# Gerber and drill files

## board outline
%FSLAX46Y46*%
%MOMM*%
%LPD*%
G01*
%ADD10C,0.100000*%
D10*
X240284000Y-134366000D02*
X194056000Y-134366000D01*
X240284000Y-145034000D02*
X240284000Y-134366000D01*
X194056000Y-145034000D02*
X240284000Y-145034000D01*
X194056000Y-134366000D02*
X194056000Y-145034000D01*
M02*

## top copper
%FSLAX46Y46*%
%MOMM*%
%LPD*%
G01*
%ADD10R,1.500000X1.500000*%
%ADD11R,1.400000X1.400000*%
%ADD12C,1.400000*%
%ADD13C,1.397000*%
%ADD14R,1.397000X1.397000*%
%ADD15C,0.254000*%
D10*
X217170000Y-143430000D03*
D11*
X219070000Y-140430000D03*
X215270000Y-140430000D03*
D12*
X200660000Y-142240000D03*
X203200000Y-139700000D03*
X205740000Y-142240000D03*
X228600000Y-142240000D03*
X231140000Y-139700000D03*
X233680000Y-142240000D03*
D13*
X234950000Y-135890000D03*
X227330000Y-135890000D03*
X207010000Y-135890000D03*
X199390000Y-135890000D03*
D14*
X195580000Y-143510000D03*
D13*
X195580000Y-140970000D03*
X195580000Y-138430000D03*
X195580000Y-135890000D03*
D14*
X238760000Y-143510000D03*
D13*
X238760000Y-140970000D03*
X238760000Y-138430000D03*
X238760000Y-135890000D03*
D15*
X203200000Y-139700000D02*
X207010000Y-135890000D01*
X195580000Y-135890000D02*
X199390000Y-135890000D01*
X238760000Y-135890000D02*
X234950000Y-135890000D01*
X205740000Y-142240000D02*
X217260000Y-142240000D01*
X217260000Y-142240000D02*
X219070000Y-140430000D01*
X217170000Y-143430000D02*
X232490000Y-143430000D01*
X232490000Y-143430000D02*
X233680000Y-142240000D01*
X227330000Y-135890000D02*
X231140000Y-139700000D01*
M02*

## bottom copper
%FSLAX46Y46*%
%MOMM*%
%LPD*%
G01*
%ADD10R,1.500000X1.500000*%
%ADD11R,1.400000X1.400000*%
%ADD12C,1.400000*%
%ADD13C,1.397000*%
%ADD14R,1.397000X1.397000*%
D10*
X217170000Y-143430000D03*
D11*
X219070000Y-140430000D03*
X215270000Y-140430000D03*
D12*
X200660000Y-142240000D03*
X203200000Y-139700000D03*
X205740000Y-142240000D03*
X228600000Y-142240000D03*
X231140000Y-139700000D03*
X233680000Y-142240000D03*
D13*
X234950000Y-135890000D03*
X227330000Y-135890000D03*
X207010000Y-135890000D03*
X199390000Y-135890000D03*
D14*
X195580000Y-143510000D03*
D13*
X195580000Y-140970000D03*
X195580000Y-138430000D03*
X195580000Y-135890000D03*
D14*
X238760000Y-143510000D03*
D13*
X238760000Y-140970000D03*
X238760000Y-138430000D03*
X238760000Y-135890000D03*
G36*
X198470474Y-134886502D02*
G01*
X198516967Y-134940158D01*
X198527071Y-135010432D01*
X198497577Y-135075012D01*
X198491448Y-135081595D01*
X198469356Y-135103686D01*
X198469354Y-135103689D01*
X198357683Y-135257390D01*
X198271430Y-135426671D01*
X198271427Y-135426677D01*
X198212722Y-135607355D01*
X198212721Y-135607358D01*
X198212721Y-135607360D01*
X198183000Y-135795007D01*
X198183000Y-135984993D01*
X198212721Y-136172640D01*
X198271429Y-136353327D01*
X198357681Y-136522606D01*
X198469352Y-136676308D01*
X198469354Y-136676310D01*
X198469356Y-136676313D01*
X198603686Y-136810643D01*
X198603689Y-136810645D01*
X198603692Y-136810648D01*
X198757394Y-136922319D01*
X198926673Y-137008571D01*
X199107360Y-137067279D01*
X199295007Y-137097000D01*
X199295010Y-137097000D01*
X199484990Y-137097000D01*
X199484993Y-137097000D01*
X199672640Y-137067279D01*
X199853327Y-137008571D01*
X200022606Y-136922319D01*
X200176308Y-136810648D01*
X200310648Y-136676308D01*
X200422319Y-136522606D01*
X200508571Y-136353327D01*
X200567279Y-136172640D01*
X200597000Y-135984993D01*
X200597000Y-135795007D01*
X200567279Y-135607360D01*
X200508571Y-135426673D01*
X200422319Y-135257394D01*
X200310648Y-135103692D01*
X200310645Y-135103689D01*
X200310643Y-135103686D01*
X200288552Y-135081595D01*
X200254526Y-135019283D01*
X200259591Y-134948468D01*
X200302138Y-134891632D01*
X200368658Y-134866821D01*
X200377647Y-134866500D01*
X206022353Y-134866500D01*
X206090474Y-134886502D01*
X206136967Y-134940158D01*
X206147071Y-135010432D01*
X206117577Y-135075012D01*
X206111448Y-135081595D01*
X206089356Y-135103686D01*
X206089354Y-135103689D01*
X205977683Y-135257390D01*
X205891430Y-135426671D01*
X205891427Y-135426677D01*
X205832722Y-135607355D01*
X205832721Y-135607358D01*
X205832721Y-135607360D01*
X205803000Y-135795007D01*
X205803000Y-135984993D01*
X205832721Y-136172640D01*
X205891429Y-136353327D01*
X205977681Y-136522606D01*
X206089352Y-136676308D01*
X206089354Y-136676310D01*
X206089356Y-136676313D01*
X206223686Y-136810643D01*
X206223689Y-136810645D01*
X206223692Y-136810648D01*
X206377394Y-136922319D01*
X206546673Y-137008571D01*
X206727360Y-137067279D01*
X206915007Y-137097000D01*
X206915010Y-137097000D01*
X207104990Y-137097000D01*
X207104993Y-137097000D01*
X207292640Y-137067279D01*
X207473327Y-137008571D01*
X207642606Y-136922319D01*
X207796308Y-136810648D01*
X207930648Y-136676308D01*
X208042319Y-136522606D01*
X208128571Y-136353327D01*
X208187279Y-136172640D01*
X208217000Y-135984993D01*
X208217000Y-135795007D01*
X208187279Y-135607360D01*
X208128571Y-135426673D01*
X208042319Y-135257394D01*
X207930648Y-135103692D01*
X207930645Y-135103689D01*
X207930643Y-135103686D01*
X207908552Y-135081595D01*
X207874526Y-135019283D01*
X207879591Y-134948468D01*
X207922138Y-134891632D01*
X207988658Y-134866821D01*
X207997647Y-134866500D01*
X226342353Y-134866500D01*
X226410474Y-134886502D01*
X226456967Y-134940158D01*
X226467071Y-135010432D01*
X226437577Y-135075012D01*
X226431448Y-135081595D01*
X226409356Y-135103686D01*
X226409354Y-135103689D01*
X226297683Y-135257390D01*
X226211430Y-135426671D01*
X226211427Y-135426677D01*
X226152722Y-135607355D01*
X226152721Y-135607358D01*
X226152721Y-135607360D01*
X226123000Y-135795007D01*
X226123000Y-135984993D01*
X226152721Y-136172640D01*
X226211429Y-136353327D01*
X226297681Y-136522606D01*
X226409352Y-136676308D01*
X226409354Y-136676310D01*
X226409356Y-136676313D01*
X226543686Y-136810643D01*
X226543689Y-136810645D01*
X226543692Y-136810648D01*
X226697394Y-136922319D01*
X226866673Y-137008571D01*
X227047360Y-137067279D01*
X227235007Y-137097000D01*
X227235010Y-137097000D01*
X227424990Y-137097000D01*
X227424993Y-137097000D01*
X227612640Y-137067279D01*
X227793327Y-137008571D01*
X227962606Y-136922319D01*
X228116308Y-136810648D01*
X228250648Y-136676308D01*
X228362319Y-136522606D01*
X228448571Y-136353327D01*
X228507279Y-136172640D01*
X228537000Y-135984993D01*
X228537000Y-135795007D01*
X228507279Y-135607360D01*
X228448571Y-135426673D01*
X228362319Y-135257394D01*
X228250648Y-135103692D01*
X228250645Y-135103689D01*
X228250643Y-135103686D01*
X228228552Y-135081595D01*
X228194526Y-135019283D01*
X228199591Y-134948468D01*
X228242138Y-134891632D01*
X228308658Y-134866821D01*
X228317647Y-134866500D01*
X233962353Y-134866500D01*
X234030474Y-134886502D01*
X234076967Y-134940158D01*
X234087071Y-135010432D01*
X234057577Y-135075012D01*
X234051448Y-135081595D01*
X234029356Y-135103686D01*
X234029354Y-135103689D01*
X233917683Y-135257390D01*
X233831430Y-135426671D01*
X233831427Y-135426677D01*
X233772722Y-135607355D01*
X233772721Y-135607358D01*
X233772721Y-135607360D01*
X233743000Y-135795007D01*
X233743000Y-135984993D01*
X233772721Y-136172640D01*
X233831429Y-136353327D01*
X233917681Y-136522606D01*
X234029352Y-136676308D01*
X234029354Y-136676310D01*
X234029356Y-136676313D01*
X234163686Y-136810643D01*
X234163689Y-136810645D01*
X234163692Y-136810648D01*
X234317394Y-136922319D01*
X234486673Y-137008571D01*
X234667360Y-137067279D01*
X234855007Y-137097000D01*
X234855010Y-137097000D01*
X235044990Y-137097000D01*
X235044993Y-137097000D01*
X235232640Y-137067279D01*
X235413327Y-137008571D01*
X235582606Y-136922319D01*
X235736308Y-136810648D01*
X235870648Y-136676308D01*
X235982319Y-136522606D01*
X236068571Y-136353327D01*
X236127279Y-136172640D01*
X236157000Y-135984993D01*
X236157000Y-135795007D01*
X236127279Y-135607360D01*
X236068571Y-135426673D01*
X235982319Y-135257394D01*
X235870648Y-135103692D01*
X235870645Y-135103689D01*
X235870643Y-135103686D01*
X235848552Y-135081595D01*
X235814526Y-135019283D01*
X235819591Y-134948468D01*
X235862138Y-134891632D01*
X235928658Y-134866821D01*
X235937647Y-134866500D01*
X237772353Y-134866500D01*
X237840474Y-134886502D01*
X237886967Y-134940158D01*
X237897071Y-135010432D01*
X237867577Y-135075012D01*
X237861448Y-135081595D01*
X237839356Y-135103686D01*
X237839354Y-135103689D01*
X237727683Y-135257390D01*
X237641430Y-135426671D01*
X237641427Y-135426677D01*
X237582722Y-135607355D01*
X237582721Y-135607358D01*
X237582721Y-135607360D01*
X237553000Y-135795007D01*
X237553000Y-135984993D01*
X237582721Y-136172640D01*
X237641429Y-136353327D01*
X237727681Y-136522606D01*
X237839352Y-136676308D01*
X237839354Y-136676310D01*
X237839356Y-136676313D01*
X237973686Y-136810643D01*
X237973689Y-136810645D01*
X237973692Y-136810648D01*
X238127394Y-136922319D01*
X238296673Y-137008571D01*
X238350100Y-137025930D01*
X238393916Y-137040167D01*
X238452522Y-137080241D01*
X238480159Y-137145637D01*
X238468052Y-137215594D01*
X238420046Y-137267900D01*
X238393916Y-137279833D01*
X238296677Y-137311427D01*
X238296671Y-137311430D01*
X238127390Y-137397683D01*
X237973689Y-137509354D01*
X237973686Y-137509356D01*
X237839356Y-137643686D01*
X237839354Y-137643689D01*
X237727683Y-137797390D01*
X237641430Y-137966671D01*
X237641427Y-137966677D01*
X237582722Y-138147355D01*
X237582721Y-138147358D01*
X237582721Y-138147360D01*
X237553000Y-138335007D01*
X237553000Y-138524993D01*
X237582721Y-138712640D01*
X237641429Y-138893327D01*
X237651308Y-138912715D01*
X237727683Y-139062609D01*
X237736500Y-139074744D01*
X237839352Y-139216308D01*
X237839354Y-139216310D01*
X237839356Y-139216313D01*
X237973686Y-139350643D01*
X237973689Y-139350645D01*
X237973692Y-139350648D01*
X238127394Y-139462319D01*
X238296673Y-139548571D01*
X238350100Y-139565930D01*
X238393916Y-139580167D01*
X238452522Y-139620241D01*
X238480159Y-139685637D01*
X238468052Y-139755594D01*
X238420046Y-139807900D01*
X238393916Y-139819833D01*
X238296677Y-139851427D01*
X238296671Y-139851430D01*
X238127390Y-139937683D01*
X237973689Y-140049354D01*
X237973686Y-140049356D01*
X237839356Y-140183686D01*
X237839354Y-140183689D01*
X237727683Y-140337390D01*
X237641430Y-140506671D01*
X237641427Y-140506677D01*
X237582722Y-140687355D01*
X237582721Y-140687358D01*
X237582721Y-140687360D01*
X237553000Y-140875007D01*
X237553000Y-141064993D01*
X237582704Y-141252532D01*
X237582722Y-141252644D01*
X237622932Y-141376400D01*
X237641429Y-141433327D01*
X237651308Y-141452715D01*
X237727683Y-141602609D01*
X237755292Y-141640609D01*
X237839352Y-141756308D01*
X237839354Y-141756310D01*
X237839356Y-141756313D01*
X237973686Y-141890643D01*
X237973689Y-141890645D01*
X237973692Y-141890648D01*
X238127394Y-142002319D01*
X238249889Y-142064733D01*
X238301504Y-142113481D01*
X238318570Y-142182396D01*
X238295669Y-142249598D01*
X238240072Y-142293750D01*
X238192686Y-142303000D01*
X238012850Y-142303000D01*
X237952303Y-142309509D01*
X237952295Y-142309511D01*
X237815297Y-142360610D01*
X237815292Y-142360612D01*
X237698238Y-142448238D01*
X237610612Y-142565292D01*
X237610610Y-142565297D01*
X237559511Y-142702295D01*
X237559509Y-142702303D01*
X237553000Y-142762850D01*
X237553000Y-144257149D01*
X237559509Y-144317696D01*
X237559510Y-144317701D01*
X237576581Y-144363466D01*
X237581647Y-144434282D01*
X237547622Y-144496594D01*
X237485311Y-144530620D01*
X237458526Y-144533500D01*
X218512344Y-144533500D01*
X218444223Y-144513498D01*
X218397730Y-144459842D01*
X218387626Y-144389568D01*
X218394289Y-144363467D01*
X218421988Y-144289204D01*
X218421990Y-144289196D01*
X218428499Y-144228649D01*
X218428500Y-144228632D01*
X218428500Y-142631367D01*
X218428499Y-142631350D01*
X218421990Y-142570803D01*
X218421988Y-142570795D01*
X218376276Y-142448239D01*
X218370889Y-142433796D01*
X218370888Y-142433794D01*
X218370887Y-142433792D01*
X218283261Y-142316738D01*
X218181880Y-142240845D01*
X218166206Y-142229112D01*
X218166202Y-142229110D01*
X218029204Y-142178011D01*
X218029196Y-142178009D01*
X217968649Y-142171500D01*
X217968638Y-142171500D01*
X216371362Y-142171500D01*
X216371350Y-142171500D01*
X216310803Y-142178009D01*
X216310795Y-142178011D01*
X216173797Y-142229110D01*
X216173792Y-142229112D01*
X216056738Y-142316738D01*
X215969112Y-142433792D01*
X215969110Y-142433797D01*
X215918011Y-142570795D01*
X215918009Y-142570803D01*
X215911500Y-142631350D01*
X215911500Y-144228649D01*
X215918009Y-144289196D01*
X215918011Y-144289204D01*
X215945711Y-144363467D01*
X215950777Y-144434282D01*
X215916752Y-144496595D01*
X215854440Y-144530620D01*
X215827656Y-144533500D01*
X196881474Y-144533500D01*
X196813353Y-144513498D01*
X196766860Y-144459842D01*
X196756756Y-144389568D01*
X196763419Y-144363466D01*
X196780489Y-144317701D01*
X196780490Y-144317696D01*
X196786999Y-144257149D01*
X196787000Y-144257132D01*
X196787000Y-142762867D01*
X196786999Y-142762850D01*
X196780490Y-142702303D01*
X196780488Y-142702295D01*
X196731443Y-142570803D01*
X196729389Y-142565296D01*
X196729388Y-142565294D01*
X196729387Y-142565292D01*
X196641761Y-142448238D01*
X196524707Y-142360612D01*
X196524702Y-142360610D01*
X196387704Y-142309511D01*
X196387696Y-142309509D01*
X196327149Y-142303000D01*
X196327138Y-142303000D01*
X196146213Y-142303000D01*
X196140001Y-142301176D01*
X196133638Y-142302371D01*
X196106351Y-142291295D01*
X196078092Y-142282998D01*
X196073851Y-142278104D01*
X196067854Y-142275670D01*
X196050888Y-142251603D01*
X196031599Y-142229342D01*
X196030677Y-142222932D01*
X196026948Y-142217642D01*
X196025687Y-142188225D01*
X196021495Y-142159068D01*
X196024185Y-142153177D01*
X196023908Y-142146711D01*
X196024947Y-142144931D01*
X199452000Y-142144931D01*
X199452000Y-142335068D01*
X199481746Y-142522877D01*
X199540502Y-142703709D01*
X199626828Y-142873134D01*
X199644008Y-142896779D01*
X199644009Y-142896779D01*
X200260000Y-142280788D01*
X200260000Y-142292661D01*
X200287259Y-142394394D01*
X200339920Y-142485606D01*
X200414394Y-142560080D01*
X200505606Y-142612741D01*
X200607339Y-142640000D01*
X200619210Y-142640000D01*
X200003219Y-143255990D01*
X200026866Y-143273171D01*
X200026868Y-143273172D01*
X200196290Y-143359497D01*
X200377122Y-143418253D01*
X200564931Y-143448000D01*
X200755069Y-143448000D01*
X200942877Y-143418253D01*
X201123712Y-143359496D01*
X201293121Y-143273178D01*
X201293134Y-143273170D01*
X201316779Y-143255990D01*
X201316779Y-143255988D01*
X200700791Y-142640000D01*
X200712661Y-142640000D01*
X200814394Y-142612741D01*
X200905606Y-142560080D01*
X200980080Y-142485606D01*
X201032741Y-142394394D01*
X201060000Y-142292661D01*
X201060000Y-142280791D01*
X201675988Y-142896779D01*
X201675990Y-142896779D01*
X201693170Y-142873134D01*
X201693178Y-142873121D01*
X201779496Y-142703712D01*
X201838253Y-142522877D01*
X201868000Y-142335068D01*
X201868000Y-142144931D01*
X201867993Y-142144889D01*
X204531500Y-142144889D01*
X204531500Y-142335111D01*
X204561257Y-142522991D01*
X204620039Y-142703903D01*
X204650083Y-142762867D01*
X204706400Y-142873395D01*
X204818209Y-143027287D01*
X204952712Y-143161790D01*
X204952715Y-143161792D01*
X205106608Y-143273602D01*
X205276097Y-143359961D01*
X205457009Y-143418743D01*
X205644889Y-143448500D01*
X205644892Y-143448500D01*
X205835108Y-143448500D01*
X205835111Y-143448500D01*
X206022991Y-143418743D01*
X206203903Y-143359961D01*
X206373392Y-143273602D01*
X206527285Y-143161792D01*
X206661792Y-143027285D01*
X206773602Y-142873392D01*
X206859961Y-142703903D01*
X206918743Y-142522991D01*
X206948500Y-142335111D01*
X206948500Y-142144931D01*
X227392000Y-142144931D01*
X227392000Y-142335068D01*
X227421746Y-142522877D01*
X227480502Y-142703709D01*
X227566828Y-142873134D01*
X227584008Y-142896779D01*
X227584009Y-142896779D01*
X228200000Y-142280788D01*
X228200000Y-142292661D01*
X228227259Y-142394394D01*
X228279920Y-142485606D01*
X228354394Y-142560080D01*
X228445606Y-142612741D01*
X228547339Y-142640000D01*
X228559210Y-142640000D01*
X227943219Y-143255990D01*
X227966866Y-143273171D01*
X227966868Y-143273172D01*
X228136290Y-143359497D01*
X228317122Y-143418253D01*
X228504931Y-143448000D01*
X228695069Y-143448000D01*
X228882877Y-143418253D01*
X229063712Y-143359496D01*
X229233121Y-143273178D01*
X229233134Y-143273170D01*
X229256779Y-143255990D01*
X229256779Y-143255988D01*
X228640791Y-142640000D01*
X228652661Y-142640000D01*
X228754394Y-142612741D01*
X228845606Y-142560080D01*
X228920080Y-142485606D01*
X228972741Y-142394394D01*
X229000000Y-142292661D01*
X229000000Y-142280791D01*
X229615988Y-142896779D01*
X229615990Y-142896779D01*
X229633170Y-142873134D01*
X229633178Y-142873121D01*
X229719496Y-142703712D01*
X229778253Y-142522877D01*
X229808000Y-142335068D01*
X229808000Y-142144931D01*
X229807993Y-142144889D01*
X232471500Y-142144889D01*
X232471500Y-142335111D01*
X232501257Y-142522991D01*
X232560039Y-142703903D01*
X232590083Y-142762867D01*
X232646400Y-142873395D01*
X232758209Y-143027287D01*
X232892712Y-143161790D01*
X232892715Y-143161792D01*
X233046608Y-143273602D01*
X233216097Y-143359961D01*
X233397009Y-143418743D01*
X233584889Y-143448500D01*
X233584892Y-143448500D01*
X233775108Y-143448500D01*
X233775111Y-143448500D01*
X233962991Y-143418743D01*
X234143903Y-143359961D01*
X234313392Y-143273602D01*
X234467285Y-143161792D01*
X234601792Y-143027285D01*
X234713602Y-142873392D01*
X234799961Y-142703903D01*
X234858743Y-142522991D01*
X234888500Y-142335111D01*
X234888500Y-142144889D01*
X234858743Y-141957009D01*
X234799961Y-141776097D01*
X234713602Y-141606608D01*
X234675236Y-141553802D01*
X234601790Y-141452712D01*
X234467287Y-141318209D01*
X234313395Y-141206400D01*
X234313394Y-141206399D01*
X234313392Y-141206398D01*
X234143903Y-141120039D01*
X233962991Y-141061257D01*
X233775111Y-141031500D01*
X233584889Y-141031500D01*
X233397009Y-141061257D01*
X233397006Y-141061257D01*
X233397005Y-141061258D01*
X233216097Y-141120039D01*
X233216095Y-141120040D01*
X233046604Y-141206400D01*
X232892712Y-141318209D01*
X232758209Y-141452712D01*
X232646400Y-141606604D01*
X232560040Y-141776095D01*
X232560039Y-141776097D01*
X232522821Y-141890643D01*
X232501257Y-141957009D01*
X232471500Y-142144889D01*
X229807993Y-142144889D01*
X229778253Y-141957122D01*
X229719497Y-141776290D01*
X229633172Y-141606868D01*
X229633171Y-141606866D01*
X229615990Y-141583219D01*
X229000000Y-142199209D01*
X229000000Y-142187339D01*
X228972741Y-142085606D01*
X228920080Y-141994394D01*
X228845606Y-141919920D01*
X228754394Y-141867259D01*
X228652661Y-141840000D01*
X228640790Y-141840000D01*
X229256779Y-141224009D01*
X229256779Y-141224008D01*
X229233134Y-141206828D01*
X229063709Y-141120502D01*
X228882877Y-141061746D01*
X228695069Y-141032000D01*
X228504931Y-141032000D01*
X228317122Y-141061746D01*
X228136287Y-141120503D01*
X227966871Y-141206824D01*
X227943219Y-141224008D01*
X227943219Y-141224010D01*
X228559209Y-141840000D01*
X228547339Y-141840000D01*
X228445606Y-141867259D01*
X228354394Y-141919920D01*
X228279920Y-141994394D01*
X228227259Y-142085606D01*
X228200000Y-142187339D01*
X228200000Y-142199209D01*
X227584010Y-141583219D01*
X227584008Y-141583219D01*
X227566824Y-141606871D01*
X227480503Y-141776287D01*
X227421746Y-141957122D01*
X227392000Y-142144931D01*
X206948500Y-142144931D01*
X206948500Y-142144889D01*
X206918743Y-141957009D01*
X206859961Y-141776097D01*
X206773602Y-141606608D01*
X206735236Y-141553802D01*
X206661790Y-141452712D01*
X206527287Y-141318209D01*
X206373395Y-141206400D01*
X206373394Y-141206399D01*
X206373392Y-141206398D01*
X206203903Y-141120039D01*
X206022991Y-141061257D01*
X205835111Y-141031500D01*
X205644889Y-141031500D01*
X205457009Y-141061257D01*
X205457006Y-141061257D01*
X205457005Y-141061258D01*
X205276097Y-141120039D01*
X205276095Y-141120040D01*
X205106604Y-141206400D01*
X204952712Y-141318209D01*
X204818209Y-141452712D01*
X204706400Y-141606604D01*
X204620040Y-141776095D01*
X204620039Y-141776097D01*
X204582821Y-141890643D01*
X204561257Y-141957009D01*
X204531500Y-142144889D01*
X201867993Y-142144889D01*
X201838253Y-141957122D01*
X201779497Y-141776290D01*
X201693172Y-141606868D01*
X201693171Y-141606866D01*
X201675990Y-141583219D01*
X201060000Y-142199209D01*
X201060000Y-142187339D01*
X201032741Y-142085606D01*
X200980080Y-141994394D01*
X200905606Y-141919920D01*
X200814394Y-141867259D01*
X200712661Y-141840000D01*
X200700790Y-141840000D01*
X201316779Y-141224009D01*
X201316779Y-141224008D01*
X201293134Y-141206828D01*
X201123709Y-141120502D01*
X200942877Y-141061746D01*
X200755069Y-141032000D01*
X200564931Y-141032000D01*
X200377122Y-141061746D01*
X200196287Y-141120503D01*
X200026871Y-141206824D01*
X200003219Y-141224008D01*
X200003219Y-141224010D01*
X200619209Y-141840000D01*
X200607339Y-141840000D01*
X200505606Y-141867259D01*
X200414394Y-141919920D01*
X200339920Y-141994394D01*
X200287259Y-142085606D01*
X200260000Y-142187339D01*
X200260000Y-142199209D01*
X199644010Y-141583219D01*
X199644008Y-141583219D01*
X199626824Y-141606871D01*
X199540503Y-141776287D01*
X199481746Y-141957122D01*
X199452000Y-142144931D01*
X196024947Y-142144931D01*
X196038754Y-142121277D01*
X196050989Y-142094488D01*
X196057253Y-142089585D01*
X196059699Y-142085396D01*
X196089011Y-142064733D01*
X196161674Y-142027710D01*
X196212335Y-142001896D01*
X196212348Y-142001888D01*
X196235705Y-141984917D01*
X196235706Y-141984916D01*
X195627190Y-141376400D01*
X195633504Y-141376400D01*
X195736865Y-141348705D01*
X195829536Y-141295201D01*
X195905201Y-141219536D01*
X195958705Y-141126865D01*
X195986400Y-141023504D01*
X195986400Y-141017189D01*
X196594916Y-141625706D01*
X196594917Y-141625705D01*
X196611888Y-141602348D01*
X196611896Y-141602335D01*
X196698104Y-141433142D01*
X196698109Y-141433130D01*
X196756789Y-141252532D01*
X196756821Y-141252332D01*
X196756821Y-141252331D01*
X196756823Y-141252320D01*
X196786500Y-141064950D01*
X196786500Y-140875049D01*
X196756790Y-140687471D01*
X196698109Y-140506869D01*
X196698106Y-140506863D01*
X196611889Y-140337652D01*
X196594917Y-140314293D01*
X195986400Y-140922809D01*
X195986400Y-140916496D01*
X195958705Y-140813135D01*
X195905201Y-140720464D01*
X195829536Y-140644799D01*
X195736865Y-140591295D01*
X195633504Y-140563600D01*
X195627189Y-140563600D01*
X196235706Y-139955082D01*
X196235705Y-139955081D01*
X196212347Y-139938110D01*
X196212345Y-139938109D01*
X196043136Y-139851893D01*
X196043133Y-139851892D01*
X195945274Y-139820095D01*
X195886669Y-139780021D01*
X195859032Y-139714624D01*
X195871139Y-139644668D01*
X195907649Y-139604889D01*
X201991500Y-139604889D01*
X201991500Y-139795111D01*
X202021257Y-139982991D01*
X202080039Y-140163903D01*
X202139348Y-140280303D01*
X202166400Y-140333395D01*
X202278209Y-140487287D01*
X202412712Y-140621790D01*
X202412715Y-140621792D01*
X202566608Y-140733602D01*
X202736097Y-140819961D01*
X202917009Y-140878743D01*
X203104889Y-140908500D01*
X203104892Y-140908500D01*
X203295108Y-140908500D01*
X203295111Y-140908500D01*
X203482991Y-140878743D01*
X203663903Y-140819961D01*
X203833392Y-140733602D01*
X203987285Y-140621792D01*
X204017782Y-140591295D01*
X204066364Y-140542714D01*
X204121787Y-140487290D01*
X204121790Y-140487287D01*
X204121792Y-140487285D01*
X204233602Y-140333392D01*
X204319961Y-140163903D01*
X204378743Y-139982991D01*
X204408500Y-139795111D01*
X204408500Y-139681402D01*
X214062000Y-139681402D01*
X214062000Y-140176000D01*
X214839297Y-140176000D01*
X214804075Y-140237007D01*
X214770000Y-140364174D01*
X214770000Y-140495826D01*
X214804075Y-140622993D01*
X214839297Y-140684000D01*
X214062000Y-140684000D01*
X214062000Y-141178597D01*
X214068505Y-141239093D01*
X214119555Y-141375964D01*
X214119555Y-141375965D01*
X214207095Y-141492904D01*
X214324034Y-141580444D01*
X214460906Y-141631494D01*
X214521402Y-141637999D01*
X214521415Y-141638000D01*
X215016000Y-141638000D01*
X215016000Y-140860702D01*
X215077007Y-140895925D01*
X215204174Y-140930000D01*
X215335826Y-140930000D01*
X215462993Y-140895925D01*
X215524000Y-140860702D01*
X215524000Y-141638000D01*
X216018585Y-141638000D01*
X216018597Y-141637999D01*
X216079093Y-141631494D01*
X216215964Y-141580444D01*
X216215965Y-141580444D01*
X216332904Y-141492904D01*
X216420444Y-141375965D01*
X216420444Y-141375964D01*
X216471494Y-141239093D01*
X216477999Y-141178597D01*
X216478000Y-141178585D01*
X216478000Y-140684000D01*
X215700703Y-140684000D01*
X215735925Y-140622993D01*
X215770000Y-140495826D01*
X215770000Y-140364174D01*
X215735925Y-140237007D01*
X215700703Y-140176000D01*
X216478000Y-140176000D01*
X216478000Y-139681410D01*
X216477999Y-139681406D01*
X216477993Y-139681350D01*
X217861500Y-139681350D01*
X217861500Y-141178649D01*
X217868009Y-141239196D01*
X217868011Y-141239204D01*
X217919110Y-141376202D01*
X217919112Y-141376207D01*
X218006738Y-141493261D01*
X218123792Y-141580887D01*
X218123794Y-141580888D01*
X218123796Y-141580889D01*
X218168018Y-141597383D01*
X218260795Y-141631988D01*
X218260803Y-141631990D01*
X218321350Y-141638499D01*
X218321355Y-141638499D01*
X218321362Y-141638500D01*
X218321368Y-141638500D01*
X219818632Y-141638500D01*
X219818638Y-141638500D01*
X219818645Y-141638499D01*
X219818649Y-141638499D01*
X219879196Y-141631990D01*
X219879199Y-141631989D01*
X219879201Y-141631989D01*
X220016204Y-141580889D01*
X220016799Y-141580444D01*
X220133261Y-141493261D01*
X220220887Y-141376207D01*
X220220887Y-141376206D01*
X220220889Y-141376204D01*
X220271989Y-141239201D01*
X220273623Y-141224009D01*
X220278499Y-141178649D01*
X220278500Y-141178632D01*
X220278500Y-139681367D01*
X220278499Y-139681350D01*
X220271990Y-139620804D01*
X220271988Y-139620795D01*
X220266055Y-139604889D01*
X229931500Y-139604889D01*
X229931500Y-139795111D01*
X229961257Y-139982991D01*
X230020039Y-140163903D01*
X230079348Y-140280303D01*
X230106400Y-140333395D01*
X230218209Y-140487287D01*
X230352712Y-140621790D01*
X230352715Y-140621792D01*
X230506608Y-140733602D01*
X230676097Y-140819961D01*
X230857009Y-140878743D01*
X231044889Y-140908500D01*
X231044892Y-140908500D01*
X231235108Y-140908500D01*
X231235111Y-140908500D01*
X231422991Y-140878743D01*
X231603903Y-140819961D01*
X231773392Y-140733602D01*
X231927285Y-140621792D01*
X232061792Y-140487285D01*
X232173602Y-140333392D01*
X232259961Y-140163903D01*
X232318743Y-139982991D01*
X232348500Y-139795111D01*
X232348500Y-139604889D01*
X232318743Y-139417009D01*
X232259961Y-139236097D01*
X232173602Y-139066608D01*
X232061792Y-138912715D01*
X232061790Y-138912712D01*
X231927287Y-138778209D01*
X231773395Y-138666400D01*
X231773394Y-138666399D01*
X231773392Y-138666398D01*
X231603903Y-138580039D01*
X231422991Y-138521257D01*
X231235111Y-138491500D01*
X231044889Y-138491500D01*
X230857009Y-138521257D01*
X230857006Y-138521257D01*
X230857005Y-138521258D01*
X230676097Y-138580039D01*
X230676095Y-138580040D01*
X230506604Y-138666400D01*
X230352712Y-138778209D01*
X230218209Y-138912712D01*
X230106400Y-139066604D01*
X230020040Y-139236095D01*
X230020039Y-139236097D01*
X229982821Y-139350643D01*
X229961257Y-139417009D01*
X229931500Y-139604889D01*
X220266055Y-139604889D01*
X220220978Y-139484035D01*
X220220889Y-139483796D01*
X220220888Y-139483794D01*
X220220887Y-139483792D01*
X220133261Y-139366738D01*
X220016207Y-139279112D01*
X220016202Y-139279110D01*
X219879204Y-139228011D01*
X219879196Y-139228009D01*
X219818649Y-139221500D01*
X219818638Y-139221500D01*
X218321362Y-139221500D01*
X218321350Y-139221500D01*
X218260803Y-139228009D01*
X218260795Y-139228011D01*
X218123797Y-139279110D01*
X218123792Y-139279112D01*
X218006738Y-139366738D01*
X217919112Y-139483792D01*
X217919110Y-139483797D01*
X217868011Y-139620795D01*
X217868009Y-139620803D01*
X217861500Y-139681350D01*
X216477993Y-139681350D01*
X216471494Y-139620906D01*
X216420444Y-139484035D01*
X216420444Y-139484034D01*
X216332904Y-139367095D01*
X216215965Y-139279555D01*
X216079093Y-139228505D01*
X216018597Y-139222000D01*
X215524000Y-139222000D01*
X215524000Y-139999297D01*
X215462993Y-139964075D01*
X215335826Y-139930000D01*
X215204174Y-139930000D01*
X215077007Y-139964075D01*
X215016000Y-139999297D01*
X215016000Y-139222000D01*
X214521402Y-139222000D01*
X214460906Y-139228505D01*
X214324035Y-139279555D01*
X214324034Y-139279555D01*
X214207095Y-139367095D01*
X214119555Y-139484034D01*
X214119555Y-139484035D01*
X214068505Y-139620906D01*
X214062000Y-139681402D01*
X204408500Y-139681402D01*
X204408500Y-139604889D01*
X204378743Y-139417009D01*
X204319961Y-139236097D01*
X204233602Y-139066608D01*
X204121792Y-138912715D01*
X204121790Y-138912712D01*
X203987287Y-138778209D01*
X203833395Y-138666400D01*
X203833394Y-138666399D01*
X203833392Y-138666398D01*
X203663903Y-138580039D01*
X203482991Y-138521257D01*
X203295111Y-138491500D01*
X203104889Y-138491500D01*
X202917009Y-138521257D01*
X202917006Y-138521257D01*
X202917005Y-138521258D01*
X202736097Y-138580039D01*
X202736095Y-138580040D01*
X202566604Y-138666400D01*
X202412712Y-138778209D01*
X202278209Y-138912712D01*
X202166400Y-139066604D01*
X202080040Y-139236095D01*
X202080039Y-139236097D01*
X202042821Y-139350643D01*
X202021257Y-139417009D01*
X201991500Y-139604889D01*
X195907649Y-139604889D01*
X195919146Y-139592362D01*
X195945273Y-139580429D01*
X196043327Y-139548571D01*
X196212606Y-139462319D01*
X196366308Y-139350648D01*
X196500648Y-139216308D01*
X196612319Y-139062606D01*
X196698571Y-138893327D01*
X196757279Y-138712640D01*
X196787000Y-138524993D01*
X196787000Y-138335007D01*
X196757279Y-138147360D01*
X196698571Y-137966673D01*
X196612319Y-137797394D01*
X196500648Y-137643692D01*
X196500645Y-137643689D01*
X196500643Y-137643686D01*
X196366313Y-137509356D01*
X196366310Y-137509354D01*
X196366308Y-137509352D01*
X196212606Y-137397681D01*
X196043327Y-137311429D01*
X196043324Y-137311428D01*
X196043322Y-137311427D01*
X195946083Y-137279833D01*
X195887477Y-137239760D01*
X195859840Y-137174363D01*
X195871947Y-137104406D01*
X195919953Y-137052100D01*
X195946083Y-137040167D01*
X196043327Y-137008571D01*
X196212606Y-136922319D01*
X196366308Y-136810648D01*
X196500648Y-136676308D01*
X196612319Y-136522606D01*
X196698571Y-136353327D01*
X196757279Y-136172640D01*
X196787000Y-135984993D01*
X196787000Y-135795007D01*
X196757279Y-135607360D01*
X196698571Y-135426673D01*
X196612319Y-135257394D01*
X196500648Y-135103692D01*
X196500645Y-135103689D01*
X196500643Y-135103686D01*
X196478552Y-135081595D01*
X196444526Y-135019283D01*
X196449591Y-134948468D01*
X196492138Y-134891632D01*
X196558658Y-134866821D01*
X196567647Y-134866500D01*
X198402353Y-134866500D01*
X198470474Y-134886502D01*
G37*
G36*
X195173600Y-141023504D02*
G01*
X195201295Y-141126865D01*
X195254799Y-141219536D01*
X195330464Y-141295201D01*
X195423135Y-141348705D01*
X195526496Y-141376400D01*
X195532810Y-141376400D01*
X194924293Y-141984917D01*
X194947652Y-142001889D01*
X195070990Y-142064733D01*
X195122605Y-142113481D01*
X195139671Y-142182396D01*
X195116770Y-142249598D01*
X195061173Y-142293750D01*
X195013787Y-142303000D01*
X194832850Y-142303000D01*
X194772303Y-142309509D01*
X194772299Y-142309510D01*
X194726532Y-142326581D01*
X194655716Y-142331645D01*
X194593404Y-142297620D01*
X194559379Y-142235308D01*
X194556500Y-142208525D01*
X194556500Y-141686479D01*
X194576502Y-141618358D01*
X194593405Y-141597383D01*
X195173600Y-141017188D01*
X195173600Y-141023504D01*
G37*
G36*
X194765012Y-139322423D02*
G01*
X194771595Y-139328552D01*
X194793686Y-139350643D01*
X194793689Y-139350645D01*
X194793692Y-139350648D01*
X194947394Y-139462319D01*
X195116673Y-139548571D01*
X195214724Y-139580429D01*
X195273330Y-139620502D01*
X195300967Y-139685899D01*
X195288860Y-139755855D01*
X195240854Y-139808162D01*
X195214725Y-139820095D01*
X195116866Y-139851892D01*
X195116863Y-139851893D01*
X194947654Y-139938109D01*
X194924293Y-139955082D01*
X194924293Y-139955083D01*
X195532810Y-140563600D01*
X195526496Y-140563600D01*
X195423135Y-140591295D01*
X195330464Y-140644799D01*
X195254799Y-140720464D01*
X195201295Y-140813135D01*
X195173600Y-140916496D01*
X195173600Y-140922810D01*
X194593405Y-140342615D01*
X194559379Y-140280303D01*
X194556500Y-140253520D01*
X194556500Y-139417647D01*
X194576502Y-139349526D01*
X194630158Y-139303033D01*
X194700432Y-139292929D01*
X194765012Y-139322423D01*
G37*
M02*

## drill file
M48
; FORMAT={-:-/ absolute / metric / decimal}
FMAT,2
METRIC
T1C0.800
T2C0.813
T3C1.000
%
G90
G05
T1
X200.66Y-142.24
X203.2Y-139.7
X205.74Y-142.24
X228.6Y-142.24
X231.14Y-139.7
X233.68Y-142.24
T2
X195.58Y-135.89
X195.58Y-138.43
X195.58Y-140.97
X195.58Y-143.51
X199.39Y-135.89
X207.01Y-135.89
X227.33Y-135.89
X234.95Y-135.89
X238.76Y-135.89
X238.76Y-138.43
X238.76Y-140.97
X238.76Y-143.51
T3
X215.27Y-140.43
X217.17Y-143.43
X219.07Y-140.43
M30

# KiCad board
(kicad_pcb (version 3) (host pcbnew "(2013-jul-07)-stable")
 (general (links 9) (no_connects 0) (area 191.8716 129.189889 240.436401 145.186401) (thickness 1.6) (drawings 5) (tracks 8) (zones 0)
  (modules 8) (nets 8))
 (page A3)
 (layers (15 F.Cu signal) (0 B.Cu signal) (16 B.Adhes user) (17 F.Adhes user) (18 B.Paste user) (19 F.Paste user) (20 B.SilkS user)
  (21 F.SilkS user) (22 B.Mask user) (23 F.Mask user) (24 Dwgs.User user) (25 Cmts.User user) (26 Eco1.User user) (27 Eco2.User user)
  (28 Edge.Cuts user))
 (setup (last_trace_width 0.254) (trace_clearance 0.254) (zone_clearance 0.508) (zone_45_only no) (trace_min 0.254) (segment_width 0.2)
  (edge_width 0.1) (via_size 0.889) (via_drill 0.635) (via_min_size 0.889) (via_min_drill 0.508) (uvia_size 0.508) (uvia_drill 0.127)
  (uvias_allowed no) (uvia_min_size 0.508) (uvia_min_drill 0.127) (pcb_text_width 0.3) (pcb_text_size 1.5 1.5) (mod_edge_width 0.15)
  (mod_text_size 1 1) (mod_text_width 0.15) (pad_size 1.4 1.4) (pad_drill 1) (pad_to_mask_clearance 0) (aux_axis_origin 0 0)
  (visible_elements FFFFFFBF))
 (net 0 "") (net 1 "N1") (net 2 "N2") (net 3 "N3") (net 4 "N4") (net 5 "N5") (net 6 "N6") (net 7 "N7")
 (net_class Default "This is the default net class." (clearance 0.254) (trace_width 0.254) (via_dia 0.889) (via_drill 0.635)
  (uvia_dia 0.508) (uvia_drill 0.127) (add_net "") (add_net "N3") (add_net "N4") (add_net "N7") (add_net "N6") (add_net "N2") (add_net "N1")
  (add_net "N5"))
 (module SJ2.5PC (layer F.Cu) (at 217.17 138.43 270)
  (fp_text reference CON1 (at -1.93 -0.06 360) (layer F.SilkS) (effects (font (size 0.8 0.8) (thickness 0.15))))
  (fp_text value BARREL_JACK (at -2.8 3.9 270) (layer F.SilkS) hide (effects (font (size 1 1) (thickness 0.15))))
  (pad 3 thru_hole rect (at 5 0 270) (size 1.5 1.5) (drill 1) (layers *.Cu *.Mask F.SilkS) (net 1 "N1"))
  (pad 2 thru_hole rect (at 2 -1.9 270) (size 1.4 1.4) (drill 1) (layers *.Cu *.Mask F.SilkS) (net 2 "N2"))
  (pad 1 thru_hole rect (at 2 1.9 270) (size 1.4 1.4) (drill 1) (layers *.Cu *.Mask F.SilkS) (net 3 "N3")))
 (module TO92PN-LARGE (layer F.Cu) (at 203.2 139.7 180)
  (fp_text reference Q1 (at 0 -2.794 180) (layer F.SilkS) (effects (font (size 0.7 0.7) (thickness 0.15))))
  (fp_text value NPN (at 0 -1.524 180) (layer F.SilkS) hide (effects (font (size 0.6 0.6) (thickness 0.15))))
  (pad 1 thru_hole circle (at 2.54 -2.54 180) (size 1.4 1.4) (drill 0.8) (layers *.Cu *.Mask F.SilkS) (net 3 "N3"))
  (pad 2 thru_hole circle (at 0 0 180) (size 1.4 1.4) (drill 0.8) (layers *.Cu *.Mask F.SilkS) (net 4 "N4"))
  (pad 3 thru_hole circle (at -2.54 -2.54 180) (size 1.4 1.4) (drill 0.8) (layers *.Cu *.Mask F.SilkS) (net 2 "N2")))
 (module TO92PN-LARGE (layer F.Cu) (at 231.14 139.7 180)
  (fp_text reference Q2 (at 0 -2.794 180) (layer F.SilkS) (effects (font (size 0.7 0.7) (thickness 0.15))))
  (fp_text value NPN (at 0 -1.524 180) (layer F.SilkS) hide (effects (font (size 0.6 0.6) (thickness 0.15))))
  (pad 1 thru_hole circle (at 2.54 -2.54 180) (size 1.4 1.4) (drill 0.8) (layers *.Cu *.Mask F.SilkS) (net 3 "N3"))
  (pad 2 thru_hole circle (at 0 0 180) (size 1.4 1.4) (drill 0.8) (layers *.Cu *.Mask F.SilkS) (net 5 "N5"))
  (pad 3 thru_hole circle (at -2.54 -2.54 180) (size 1.4 1.4) (drill 0.8) (layers *.Cu *.Mask F.SilkS) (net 1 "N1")))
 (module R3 (layer F.Cu) (at 231.14 135.89 180) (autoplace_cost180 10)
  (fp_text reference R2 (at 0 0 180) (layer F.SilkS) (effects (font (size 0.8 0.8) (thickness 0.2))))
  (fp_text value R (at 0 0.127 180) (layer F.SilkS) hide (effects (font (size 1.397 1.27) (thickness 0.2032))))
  (pad 1 thru_hole circle (at -3.81 0 180) (size 1.397 1.397) (drill 0.8128) (layers *.Cu *.Mask F.SilkS) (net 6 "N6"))
  (pad 2 thru_hole circle (at 3.81 0 180) (size 1.397 1.397) (drill 0.8128) (layers *.Cu *.Mask F.SilkS) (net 5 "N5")))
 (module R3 (layer F.Cu) (at 203.2 135.89 180) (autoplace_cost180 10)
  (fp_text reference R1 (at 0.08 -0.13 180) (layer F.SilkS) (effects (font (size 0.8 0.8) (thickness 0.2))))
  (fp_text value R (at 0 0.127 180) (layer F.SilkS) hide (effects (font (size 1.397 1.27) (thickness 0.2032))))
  (pad 1 thru_hole circle (at -3.81 0 180) (size 1.397 1.397) (drill 0.8128) (layers *.Cu *.Mask F.SilkS) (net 4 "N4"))
  (pad 2 thru_hole circle (at 3.81 0 180) (size 1.397 1.397) (drill 0.8128) (layers *.Cu *.Mask F.SilkS) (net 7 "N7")))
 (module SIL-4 (layer F.Cu) (at 195.58 139.7 90)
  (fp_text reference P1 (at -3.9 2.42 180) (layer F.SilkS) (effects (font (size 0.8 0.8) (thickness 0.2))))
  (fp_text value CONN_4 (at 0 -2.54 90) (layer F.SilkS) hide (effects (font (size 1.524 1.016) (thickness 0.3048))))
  (pad 1 thru_hole rect (at -3.81 0 90) (size 1.397 1.397) (drill 0.8128) (layers *.Cu *.Mask F.SilkS))
  (pad 2 thru_hole circle (at -1.27 0 90) (size 1.397 1.397) (drill 0.8128) (layers *.Cu *.Mask F.SilkS) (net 3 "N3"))
  (pad 3 thru_hole circle (at 1.27 0 90) (size 1.397 1.397) (drill 0.8128) (layers *.Cu *.Mask F.SilkS))
  (pad 4 thru_hole circle (at 3.81 0 90) (size 1.397 1.397) (drill 0.8128) (layers *.Cu *.Mask F.SilkS) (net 7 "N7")))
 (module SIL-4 (layer F.Cu) (at 238.76 139.7 90)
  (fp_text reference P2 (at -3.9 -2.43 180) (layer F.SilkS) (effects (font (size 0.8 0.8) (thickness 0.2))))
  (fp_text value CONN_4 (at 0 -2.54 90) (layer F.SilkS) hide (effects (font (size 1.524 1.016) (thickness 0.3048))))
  (pad 1 thru_hole rect (at -3.81 0 90) (size 1.397 1.397) (drill 0.8128) (layers *.Cu *.Mask F.SilkS))
  (pad 2 thru_hole circle (at -1.27 0 90) (size 1.397 1.397) (drill 0.8128) (layers *.Cu *.Mask F.SilkS))
  (pad 3 thru_hole circle (at 1.27 0 90) (size 1.397 1.397) (drill 0.8128) (layers *.Cu *.Mask F.SilkS))
  (pad 4 thru_hole circle (at 3.81 0 90) (size 1.397 1.397) (drill 0.8128) (layers *.Cu *.Mask F.SilkS) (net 6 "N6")))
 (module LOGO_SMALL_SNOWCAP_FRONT (layer F.Cu) (at 210.82 139.446 90)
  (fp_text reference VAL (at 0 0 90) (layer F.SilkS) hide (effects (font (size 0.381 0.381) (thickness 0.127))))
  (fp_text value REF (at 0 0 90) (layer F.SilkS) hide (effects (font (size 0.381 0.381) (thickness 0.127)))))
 (gr_line (start 240.284 134.366) (end 194.056 134.366) (angle 90) (layer Edge.Cuts) (width 0.1))
 (gr_line (start 240.284 145.034) (end 240.284 134.366) (angle 90) (layer Edge.Cuts) (width 0.1))
 (gr_line (start 194.056 145.034) (end 240.284 145.034) (angle 90) (layer Edge.Cuts) (width 0.1))
 (gr_line (start 194.056 134.366) (end 194.056 145.034) (angle 90) (layer Edge.Cuts) (width 0.1))
 (segment (start 203.2 139.7) (end 207.01 135.89) (width 0.254) (layer F.Cu) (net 4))
 (segment (start 195.58 135.89) (end 199.39 135.89) (width 0.254) (layer F.Cu) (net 7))
 (segment (start 238.76 135.89) (end 234.95 135.89) (width 0.254) (layer F.Cu) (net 6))
 (segment (start 205.74 142.24) (end 217.26 142.24) (width 0.254) (layer F.Cu) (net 2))
 (segment (start 217.26 142.24) (end 219.07 140.43) (width 0.254) (layer F.Cu) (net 2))
 (segment (start 217.17 143.43) (end 232.49 143.43) (width 0.254) (layer F.Cu) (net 1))
 (segment (start 232.49 143.43) (end 233.68 142.24) (width 0.254) (layer F.Cu) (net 1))
 (segment (start 227.33 135.89) (end 231.14 139.7) (width 0.254) (layer F.Cu) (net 5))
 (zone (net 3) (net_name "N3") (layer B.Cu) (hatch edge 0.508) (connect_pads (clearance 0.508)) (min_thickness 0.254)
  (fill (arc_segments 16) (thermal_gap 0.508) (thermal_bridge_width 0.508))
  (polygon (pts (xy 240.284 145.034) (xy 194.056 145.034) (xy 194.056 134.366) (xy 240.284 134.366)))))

